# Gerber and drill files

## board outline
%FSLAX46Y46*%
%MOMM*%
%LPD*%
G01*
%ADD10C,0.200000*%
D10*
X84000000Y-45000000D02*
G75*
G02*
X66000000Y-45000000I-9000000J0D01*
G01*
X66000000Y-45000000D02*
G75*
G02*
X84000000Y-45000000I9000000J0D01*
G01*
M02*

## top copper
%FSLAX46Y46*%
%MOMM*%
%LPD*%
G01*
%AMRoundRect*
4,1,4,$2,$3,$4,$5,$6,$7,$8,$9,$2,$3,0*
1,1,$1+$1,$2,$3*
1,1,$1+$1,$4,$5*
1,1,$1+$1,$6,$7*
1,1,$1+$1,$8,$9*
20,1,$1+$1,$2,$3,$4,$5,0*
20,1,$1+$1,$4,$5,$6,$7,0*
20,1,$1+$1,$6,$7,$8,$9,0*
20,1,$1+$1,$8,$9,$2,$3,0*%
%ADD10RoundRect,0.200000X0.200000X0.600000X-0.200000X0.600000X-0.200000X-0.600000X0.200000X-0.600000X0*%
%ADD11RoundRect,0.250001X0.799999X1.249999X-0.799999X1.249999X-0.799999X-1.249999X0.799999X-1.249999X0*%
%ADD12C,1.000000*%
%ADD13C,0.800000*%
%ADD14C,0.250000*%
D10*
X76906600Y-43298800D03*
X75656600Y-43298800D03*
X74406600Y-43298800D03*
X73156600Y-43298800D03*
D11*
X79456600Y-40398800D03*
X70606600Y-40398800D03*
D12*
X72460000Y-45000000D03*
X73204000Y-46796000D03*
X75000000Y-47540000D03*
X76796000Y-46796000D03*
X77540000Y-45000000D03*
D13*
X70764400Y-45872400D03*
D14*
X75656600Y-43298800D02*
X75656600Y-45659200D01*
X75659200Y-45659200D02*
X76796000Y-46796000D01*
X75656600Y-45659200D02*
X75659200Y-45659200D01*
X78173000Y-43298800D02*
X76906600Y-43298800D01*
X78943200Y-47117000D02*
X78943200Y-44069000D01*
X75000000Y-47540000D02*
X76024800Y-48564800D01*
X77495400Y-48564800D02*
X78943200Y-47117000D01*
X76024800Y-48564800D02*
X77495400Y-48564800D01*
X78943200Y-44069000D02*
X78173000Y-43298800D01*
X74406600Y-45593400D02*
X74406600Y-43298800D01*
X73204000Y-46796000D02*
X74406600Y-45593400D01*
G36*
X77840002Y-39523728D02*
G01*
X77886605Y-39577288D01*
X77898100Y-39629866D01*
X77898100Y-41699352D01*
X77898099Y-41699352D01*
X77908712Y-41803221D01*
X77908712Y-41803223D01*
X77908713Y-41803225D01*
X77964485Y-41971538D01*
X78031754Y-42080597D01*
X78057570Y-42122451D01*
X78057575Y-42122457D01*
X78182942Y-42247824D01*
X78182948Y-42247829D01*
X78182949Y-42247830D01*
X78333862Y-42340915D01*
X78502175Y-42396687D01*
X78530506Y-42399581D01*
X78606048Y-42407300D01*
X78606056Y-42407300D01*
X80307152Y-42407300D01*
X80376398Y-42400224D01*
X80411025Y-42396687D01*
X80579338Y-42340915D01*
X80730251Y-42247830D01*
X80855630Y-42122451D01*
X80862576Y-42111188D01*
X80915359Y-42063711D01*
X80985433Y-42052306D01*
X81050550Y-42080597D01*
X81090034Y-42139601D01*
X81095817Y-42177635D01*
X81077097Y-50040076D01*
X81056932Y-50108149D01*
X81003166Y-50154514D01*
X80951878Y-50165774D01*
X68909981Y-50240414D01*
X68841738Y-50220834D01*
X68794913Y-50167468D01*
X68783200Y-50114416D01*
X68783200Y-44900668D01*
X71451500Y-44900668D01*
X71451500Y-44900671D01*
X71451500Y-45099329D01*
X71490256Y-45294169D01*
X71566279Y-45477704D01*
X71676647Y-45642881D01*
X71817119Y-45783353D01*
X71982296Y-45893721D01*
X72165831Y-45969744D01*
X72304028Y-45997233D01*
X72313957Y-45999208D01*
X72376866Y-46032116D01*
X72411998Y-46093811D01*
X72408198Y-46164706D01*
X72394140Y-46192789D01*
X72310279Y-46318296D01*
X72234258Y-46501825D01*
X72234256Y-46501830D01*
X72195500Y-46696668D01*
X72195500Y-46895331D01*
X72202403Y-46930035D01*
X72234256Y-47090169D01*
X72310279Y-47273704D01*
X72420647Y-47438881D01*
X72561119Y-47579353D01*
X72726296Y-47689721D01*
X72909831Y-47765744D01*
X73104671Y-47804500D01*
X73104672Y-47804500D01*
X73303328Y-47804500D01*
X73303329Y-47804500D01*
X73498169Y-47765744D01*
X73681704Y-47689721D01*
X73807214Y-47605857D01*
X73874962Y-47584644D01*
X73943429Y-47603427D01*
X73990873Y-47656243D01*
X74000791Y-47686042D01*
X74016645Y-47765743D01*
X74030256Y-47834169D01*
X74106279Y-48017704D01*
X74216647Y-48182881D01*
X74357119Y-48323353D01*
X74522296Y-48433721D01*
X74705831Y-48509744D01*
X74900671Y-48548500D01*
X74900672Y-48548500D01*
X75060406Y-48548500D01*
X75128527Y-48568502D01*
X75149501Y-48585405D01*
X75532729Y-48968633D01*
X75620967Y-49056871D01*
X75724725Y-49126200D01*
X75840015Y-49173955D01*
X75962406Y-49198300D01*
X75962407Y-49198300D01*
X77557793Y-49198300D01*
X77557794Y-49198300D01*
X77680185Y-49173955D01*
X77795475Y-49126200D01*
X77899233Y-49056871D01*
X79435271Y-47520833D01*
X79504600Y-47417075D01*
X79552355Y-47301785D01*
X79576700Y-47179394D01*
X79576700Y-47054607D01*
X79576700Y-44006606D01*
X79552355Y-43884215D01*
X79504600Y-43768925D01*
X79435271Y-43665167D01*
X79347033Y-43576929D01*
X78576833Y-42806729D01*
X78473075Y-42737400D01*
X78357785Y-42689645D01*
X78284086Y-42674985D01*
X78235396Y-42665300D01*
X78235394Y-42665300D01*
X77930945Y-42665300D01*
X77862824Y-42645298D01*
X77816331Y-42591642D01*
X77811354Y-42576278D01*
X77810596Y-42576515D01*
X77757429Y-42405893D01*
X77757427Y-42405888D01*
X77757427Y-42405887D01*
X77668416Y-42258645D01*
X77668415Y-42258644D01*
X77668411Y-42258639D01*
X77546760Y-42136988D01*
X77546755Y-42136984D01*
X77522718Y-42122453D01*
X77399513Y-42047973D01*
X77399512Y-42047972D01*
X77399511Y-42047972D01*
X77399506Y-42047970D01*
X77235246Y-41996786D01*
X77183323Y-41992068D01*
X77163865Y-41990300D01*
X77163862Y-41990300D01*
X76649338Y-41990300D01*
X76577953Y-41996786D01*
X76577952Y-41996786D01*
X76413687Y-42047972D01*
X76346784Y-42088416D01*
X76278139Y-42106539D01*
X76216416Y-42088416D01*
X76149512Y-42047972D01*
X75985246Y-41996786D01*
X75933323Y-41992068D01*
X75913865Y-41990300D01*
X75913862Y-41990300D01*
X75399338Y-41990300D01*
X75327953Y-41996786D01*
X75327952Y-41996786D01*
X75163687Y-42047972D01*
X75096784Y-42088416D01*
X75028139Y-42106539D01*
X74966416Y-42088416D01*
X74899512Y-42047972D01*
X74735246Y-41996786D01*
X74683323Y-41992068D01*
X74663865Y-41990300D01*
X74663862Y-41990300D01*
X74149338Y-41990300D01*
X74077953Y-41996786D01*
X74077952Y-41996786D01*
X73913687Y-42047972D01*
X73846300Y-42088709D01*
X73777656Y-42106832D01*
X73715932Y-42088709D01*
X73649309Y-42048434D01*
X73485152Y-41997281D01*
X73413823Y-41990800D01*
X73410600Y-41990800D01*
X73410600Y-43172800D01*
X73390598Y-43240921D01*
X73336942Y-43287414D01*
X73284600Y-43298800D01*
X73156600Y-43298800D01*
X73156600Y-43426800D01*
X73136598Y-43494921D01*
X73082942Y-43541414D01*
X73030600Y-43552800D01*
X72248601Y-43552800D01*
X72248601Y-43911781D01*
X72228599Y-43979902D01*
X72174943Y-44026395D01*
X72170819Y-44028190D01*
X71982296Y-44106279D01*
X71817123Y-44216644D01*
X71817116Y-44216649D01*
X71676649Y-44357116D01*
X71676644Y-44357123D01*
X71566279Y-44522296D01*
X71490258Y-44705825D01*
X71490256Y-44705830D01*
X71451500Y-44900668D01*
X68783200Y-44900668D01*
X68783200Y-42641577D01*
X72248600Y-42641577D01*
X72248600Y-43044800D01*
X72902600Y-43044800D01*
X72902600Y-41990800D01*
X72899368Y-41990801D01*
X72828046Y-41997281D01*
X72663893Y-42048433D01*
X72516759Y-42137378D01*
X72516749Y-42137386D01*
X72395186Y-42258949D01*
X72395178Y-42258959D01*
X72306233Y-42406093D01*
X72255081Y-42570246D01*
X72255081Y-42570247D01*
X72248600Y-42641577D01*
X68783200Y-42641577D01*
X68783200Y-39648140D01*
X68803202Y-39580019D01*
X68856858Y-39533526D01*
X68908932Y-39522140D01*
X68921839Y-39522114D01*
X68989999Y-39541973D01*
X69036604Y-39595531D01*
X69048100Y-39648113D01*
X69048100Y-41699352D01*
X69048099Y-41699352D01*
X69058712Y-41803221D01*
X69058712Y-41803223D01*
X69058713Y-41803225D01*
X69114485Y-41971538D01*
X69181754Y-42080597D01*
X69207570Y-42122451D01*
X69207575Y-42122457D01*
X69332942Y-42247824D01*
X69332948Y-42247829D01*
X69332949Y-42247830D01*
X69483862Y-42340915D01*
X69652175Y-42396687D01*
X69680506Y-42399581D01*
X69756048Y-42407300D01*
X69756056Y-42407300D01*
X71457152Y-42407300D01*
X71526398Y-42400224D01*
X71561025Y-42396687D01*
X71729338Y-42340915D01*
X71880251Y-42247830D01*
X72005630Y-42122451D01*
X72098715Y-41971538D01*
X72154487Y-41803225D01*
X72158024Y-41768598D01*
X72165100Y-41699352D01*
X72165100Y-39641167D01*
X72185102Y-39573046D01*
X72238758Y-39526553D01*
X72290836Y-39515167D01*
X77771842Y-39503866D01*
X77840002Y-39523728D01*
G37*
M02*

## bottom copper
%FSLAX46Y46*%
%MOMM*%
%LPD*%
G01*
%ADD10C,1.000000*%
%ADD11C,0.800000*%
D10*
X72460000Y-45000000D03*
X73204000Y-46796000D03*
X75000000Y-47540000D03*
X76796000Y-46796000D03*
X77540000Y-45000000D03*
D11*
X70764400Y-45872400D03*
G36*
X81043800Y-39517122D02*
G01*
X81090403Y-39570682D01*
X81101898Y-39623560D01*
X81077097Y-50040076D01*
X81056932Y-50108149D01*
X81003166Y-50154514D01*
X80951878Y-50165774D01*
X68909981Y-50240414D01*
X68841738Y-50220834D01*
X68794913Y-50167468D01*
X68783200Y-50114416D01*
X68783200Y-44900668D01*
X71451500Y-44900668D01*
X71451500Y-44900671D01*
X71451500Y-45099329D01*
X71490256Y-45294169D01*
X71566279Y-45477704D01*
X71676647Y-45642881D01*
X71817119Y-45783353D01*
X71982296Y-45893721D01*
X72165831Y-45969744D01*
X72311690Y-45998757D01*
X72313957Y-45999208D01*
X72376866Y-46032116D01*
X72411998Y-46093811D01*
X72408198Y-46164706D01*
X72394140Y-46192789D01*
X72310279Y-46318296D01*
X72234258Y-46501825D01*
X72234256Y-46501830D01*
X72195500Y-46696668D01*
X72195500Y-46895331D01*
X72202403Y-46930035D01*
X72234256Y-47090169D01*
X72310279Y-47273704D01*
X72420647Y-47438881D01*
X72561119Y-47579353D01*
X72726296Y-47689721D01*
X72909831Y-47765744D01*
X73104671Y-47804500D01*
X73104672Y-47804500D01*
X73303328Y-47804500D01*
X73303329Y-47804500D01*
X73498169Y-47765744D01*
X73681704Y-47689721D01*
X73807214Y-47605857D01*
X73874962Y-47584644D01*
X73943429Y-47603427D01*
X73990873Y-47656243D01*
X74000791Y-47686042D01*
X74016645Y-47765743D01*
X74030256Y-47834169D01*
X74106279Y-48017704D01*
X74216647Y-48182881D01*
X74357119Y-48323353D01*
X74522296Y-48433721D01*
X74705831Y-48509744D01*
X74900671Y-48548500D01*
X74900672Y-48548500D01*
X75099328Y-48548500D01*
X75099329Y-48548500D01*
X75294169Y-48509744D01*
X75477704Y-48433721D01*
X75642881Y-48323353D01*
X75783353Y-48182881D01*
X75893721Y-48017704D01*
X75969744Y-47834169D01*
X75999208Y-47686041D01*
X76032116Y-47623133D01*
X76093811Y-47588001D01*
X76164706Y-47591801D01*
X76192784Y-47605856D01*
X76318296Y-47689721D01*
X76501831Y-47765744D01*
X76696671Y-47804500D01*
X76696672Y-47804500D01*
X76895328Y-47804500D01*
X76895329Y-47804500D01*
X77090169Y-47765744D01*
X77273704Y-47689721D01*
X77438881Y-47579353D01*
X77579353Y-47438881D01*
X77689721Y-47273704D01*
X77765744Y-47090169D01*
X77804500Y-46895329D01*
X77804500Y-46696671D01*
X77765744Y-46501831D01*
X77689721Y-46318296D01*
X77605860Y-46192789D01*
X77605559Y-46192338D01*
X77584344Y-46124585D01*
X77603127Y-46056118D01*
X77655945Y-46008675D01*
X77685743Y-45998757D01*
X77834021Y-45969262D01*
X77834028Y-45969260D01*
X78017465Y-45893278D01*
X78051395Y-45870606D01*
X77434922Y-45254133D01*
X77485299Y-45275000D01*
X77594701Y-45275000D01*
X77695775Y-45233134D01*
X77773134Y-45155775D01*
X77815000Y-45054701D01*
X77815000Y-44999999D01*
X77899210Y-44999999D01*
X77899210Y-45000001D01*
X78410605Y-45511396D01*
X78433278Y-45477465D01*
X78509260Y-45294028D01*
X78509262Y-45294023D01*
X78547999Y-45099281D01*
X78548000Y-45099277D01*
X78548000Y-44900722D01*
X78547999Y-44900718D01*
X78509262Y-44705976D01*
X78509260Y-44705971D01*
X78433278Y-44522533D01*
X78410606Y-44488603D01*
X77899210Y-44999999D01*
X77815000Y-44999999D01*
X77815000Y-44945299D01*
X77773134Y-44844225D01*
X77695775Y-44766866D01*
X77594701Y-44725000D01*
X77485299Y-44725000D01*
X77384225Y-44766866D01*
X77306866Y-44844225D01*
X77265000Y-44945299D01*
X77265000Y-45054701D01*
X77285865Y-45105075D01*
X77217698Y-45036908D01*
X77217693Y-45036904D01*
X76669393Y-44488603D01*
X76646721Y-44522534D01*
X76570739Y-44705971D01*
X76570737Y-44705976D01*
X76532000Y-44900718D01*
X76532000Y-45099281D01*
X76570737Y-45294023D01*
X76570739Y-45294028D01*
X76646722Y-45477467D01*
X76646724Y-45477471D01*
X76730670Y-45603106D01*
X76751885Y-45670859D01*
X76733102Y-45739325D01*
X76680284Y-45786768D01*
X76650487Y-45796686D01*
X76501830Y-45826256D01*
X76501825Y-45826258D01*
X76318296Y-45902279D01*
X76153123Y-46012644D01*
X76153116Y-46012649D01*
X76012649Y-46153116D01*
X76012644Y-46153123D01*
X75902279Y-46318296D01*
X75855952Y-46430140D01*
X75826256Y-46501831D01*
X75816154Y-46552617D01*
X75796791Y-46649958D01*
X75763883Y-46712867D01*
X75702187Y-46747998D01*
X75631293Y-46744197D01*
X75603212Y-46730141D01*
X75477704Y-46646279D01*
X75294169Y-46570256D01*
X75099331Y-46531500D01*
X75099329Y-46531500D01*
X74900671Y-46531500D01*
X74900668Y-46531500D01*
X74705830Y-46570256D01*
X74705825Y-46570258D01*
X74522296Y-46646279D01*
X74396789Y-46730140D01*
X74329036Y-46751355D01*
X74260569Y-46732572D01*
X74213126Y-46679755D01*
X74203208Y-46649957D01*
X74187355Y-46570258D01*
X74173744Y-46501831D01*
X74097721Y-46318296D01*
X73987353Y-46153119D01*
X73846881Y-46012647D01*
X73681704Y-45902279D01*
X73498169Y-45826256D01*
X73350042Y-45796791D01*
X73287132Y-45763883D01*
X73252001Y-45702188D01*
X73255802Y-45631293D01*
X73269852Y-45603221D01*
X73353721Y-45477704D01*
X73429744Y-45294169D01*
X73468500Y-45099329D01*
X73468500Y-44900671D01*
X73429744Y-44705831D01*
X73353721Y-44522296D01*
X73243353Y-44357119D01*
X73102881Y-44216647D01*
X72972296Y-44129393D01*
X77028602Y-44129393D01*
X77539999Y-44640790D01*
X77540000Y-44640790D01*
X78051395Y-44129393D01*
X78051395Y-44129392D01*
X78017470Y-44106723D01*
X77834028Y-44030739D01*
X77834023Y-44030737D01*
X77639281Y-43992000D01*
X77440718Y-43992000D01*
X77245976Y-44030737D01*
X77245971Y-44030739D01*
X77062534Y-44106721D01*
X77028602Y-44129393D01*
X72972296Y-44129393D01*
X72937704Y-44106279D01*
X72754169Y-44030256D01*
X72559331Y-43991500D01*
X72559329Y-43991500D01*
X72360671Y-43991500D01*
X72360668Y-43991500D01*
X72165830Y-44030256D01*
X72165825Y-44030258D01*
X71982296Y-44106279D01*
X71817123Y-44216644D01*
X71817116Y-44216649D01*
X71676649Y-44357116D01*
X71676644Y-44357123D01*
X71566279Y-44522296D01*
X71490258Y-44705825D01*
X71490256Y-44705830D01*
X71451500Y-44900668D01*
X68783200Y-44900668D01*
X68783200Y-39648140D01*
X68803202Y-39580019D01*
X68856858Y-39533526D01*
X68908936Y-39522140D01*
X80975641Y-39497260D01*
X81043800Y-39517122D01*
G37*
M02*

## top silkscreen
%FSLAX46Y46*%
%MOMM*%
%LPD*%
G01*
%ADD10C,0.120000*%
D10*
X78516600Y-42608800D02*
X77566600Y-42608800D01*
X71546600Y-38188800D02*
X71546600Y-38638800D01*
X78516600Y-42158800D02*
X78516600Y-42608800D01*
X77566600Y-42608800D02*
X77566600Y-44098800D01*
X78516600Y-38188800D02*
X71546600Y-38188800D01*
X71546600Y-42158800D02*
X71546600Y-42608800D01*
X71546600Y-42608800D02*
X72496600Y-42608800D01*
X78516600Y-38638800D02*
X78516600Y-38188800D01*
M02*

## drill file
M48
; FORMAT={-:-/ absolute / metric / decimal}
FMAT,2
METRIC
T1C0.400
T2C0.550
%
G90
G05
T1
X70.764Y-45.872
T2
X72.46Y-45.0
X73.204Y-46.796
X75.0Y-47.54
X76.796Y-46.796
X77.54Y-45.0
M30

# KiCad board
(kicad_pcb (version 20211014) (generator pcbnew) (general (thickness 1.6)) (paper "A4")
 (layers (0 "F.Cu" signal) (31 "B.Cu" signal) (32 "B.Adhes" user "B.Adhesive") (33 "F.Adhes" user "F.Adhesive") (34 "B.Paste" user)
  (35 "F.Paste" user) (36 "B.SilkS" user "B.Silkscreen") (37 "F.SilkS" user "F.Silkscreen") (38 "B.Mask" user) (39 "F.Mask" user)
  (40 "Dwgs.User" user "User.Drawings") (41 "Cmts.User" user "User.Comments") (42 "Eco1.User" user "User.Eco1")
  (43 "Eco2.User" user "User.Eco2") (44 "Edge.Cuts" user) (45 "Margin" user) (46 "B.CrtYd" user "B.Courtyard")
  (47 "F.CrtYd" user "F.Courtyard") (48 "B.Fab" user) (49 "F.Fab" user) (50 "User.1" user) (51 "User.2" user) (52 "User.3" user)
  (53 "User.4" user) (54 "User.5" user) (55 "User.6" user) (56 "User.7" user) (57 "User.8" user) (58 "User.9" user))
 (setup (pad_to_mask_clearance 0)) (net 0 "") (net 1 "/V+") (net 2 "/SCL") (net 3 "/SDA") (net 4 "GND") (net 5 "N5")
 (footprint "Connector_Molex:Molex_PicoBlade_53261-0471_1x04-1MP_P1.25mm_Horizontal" (layer "F.Cu") (at 75.0316 40.8988 180)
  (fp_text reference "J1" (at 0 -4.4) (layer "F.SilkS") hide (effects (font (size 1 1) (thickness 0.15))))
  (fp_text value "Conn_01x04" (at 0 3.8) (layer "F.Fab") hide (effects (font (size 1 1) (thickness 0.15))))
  (fp_line (start -3.485 -1.71) (end -2.535 -1.71) (layer "F.SilkS") (width 0.12))
  (fp_line (start 3.485 2.71) (end 3.485 2.26) (layer "F.SilkS") (width 0.12))
  (fp_line (start -3.485 -1.26) (end -3.485 -1.71) (layer "F.SilkS") (width 0.12))
  (fp_line (start -2.535 -1.71) (end -2.535 -3.2) (layer "F.SilkS") (width 0.12))
  (fp_line (start -3.485 2.71) (end 3.485 2.71) (layer "F.SilkS") (width 0.12))
  (fp_line (start 3.485 -1.26) (end 3.485 -1.71) (layer "F.SilkS") (width 0.12))
  (fp_line (start 3.485 -1.71) (end 2.535 -1.71) (layer "F.SilkS") (width 0.12))
  (fp_line (start -3.485 2.26) (end -3.485 2.71) (layer "F.SilkS") (width 0.12))
  (pad "1" smd roundrect (at -1.875 -2.4 180) (size 0.8 1.6) (layers "F.Cu" "F.Paste" "F.Mask") (roundrect_rratio 0.25) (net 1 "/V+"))
  (pad "2" smd roundrect (at -0.625 -2.4 180) (size 0.8 1.6) (layers "F.Cu" "F.Paste" "F.Mask") (roundrect_rratio 0.25) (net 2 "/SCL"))
  (pad "3" smd roundrect (at 0.625 -2.4 180) (size 0.8 1.6) (layers "F.Cu" "F.Paste" "F.Mask") (roundrect_rratio 0.25) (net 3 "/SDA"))
  (pad "4" smd roundrect (at 1.875 -2.4 180) (size 0.8 1.6) (layers "F.Cu" "F.Paste" "F.Mask") (roundrect_rratio 0.25) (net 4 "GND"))
  (pad "MP" smd roundrect (at -4.425 0.5 180) (size 2.1 3) (layers "F.Cu" "F.Paste" "F.Mask") (roundrect_rratio 0.119048))
  (pad "MP" smd roundrect (at 4.425 0.5 180) (size 2.1 3) (layers "F.Cu" "F.Paste" "F.Mask") (roundrect_rratio 0.119048)))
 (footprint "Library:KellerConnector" (layer "F.Cu") (at 75 45)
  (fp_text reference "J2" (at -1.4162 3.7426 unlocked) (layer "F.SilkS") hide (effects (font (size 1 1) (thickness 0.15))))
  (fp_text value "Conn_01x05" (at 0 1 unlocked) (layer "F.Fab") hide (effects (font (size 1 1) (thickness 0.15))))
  (pad "1" thru_hole circle (at -2.54 0) (size 1 1) (drill 0.55) (layers *.Cu *.Mask) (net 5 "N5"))
  (pad "2" thru_hole circle (at -1.796 1.796) (size 1 1) (drill 0.55) (layers *.Cu *.Mask) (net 3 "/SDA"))
  (pad "3" thru_hole circle (at 0 2.54) (size 1 1) (drill 0.55) (layers *.Cu *.Mask) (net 1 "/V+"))
  (pad "4" thru_hole circle (at 1.796 1.796) (size 1 1) (drill 0.55) (layers *.Cu *.Mask) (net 2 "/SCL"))
  (pad "5" thru_hole circle (at 2.54 0) (size 1 1) (drill 0.55) (layers *.Cu *.Mask) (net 4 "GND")))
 (gr_circle (center 75 45) (end 84 45) (layer "Edge.Cuts") (width 0.2) (fill none))
 (segment (start 75.6566 43.2988) (end 75.6566 45.6592) (width 0.25) (layer "F.Cu") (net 2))
 (segment (start 75.6592 45.6592) (end 76.796 46.796) (width 0.25) (layer "F.Cu") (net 2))
 (segment (start 75.6566 45.6592) (end 75.6592 45.6592) (width 0.25) (layer "F.Cu") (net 2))
 (segment (start 78.173 43.2988) (end 76.9066 43.2988) (width 0.25) (layer "F.Cu") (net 1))
 (segment (start 78.9432 47.117) (end 78.9432 44.069) (width 0.25) (layer "F.Cu") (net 1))
 (segment (start 75 47.54) (end 76.0248 48.5648) (width 0.25) (layer "F.Cu") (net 1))
 (segment (start 77.4954 48.5648) (end 78.9432 47.117) (width 0.25) (layer "F.Cu") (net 1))
 (segment (start 76.0248 48.5648) (end 77.4954 48.5648) (width 0.25) (layer "F.Cu") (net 1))
 (segment (start 78.9432 44.069) (end 78.173 43.2988) (width 0.25) (layer "F.Cu") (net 1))
 (segment (start 74.4066 45.5934) (end 74.4066 43.2988) (width 0.25) (layer "F.Cu") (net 3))
 (segment (start 73.204 46.796) (end 74.4066 45.5934) (width 0.25) (layer "F.Cu") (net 3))
 (via (at 70.7644 45.8724) (size 0.8) (drill 0.4) (layers "F.Cu" "B.Cu") (free) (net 4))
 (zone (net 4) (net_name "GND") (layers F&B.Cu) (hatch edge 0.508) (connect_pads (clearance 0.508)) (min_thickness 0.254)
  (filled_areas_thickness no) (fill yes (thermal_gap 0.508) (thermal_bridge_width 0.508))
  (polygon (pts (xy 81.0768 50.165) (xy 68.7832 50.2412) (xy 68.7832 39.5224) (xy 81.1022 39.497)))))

